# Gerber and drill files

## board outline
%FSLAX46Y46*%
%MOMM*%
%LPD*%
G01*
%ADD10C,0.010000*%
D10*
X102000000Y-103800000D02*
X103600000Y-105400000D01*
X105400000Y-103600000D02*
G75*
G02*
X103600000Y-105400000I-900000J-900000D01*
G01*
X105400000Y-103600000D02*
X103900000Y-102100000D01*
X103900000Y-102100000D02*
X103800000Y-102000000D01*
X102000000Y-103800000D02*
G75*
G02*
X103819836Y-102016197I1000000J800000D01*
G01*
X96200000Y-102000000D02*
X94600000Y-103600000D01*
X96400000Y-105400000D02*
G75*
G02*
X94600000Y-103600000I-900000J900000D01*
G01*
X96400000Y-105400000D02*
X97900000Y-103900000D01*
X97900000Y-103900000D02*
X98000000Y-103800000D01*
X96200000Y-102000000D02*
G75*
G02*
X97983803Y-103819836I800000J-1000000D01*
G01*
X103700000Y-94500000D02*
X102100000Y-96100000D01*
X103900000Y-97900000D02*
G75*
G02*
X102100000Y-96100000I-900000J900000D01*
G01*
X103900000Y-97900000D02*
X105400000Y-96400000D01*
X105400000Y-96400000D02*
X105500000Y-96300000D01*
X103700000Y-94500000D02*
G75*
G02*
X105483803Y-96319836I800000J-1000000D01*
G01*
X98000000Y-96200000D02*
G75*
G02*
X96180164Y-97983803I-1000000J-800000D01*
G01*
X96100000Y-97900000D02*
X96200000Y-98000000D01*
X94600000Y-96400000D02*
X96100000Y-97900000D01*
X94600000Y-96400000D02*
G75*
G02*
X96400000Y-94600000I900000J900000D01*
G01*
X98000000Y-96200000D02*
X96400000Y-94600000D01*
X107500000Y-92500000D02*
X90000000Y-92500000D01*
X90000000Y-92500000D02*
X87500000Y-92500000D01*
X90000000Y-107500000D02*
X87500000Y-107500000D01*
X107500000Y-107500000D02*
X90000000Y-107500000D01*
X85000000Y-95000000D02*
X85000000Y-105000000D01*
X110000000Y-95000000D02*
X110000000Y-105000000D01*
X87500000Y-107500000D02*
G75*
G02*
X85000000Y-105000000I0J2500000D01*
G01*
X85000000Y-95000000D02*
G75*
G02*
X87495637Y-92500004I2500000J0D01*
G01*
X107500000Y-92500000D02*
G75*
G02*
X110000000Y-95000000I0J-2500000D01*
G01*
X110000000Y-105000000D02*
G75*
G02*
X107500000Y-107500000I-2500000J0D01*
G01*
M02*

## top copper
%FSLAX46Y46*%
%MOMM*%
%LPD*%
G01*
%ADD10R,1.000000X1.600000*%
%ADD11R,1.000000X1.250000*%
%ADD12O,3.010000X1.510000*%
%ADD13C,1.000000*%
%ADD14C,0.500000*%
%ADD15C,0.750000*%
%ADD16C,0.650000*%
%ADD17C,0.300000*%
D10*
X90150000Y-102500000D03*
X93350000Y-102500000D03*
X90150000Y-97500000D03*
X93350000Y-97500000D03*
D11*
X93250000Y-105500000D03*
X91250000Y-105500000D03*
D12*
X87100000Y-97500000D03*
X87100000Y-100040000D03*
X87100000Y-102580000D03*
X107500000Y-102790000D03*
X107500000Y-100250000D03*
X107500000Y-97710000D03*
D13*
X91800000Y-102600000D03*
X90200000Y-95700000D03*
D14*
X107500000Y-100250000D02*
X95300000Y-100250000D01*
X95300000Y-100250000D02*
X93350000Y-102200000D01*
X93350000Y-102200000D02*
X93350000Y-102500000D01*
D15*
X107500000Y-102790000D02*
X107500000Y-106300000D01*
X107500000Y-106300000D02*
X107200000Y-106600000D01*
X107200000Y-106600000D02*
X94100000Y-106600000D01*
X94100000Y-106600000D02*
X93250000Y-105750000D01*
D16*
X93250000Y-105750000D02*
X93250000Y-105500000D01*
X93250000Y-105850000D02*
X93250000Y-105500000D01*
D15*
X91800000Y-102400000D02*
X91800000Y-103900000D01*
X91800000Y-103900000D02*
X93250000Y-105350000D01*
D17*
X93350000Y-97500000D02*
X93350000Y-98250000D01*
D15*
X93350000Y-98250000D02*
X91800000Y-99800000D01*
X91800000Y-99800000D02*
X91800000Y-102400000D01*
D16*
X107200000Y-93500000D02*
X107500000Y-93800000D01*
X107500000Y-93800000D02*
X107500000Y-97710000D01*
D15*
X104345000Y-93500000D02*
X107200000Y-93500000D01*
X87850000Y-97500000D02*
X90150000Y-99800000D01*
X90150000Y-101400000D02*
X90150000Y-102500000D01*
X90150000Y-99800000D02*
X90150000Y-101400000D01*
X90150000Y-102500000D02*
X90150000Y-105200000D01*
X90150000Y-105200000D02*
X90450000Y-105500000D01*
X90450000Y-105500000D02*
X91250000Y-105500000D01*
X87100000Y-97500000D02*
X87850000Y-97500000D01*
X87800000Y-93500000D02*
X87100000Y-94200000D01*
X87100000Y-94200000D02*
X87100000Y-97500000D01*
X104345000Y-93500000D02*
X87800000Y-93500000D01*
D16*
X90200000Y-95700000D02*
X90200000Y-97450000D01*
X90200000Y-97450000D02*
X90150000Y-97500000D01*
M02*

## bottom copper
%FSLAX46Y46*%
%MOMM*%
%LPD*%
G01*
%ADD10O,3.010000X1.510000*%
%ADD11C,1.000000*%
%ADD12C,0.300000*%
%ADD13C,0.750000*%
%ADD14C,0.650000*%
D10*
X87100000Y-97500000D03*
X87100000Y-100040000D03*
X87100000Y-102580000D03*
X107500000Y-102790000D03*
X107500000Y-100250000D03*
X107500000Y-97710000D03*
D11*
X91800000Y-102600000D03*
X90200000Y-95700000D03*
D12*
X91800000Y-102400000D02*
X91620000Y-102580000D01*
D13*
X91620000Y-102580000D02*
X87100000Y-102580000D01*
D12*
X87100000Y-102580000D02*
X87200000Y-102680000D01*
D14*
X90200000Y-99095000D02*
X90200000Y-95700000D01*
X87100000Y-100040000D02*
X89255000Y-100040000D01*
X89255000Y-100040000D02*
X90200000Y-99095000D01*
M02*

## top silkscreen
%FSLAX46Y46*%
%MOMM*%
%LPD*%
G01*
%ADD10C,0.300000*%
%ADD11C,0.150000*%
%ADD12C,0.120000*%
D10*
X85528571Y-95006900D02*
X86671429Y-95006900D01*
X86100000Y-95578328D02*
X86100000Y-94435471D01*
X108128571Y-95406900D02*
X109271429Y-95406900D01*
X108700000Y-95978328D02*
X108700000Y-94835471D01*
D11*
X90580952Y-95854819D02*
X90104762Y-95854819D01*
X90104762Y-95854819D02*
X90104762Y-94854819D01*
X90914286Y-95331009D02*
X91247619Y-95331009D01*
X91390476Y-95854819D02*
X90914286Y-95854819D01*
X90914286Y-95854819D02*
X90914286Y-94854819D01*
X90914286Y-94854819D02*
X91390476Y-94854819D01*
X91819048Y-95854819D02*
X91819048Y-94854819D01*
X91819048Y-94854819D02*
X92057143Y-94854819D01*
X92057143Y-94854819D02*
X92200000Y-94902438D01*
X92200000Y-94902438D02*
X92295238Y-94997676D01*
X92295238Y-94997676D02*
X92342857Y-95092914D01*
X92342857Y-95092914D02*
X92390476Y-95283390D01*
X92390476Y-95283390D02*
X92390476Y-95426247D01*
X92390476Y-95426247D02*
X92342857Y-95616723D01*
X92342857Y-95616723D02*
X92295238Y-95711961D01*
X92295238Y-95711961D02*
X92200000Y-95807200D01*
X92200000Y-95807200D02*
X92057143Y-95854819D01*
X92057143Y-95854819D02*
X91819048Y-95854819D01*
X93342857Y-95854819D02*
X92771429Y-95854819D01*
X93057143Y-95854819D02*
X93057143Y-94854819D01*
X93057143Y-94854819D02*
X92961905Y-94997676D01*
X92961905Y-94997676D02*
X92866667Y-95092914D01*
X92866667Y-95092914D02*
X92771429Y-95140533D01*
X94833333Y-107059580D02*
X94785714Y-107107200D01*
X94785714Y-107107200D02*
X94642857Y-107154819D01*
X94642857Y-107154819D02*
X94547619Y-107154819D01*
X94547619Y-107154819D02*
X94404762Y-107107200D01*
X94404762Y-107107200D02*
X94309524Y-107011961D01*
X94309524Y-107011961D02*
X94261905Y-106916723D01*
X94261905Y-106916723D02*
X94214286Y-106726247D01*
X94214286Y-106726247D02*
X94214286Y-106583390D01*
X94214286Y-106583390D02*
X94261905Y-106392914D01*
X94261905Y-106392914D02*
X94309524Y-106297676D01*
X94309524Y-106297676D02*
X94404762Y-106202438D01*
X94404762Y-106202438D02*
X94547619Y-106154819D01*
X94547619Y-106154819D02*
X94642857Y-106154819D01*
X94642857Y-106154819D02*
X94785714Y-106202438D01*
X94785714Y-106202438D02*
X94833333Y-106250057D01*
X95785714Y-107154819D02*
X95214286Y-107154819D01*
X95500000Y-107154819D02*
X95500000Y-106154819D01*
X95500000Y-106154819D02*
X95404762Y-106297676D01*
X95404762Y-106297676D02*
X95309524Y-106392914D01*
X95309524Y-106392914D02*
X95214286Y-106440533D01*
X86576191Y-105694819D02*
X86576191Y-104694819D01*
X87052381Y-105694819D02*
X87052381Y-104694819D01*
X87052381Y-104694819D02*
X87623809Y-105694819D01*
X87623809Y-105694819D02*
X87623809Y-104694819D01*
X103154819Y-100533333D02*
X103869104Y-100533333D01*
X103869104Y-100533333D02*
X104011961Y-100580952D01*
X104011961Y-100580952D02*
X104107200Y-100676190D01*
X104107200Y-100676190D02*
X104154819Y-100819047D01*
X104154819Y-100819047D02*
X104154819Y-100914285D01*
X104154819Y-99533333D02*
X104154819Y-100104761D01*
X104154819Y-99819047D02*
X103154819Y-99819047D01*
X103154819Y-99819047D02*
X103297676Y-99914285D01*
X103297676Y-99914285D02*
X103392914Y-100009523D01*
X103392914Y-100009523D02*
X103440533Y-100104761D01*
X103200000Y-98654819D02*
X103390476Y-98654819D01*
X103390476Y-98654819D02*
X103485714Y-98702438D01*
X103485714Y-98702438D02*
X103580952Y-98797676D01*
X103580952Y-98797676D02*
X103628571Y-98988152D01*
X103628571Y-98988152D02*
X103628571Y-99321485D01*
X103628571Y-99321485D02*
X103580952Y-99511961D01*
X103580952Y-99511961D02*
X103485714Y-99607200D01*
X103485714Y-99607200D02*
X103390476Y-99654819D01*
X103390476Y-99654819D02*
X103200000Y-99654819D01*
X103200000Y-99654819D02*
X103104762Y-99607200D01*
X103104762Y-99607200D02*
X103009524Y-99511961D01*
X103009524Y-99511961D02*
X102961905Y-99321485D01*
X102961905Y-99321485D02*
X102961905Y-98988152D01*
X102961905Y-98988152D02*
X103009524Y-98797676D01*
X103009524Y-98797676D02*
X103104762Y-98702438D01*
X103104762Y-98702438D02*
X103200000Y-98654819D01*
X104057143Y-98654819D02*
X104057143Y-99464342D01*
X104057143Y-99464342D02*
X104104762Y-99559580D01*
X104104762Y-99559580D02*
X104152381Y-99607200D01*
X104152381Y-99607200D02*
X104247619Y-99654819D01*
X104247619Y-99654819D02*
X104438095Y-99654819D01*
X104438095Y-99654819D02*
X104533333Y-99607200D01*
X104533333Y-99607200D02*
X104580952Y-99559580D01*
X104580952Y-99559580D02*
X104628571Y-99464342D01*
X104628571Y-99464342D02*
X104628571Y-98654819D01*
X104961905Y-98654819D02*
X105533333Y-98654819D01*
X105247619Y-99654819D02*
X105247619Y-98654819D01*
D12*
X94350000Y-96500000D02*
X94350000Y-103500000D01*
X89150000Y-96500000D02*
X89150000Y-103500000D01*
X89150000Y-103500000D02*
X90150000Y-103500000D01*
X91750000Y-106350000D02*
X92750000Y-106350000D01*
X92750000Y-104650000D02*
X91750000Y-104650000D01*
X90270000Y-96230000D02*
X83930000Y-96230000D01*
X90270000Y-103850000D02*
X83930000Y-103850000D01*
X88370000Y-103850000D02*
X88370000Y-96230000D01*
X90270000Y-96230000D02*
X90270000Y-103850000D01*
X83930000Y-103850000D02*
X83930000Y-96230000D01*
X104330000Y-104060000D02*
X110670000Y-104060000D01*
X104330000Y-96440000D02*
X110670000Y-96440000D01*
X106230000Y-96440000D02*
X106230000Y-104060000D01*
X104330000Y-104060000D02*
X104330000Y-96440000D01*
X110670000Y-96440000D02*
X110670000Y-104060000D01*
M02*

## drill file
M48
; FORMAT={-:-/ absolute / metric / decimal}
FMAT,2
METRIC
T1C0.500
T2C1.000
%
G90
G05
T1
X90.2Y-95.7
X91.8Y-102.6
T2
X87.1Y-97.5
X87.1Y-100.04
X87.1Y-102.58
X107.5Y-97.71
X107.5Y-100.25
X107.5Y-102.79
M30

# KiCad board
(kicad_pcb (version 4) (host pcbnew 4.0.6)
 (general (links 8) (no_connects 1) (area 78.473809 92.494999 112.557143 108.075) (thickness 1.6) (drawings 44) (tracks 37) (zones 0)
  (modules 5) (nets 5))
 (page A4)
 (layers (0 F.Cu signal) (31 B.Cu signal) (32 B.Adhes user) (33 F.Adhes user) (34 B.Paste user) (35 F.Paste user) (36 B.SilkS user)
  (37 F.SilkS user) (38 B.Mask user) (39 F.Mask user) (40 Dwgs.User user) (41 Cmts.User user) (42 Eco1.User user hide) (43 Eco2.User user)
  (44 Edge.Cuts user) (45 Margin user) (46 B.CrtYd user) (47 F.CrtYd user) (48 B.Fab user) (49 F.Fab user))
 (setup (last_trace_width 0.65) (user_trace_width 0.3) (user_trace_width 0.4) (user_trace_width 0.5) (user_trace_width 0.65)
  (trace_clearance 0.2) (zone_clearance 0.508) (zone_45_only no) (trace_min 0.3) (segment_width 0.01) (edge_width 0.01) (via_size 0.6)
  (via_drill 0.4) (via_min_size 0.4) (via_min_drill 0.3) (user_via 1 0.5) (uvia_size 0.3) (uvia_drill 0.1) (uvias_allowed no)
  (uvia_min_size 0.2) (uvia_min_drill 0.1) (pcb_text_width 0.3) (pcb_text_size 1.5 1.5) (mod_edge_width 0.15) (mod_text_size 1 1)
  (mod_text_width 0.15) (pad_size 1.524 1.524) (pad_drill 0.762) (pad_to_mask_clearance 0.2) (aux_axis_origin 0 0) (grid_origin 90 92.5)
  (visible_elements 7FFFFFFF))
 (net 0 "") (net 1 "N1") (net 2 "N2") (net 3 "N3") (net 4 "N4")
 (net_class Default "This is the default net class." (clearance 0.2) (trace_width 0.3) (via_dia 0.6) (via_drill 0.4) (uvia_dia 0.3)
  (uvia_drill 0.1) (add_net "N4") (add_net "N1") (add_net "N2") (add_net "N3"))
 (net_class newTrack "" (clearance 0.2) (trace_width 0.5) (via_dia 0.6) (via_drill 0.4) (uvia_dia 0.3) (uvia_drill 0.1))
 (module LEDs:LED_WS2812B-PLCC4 (layer F.Cu) (at 91.75 100 270)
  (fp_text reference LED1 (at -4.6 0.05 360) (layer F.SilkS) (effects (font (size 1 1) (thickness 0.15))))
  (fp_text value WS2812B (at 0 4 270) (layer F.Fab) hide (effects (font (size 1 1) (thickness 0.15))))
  (fp_line (start -3.5 -2.6) (end 3.5 -2.6) (layer F.SilkS) (width 0.12))
  (fp_line (start -3.5 2.6) (end 3.5 2.6) (layer F.SilkS) (width 0.12))
  (fp_line (start 3.5 2.6) (end 3.5 1.6) (layer F.SilkS) (width 0.12))
  (pad 3 smd rect (at 2.5 1.6 270) (size 1.6 1) (layers F.Cu F.Paste F.Mask) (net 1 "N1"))
  (pad 4 smd rect (at 2.5 -1.6 270) (size 1.6 1) (layers F.Cu F.Paste F.Mask) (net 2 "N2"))
  (pad 2 smd rect (at -2.5 1.6 270) (size 1.6 1) (layers F.Cu F.Paste F.Mask) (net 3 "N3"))
  (pad 1 smd rect (at -2.5 -1.6 270) (size 1.6 1) (layers F.Cu F.Paste F.Mask) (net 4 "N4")))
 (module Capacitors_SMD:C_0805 (layer F.Cu) (at 92.25 105.5 180)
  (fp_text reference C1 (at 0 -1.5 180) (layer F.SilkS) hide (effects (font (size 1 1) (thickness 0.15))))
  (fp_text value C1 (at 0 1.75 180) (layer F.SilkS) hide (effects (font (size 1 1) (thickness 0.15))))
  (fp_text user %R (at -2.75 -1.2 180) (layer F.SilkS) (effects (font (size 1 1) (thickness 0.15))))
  (fp_line (start 0.5 -0.85) (end -0.5 -0.85) (layer F.SilkS) (width 0.12))
  (fp_line (start -0.5 0.85) (end 0.5 0.85) (layer F.SilkS) (width 0.12))
  (pad 1 smd rect (at -1 0 180) (size 1 1.25) (layers F.Cu F.Paste F.Mask) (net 4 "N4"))
  (pad 2 smd rect (at 1 0 180) (size 1 1.25) (layers F.Cu F.Paste F.Mask) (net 1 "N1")))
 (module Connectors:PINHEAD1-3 (layer F.Cu) (at 87.1 97.5 270)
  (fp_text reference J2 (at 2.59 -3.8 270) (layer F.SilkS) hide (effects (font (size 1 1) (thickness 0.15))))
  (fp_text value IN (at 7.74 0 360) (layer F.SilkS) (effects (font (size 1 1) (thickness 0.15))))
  (fp_line (start -1.27 -3.17) (end -1.27 3.17) (layer F.SilkS) (width 0.12))
  (fp_line (start 6.35 -3.17) (end 6.35 3.17) (layer F.SilkS) (width 0.12))
  (fp_line (start 6.35 -1.27) (end -1.27 -1.27) (layer F.SilkS) (width 0.12))
  (fp_line (start -1.27 -3.17) (end 6.35 -3.17) (layer F.SilkS) (width 0.12))
  (fp_line (start 6.35 3.17) (end -1.27 3.17) (layer F.SilkS) (width 0.12))
  (pad 1 thru_hole oval (at 0 0 270) (size 1.51 3.01) (drill 1) (layers *.Cu *.Mask) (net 1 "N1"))
  (pad 2 thru_hole oval (at 2.54 0 270) (size 1.51 3.01) (drill 1) (layers *.Cu *.Mask) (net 3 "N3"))
  (pad 3 thru_hole oval (at 5.08 0 270) (size 1.51 3.01) (drill 1) (layers *.Cu *.Mask) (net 4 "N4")))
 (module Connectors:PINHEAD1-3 (layer F.Cu) (at 107.5 102.79 90)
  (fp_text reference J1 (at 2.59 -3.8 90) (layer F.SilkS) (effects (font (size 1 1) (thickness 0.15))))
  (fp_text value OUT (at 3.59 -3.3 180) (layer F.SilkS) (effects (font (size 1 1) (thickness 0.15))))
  (fp_line (start -1.27 -3.17) (end -1.27 3.17) (layer F.SilkS) (width 0.12))
  (fp_line (start 6.35 -3.17) (end 6.35 3.17) (layer F.SilkS) (width 0.12))
  (fp_line (start 6.35 -1.27) (end -1.27 -1.27) (layer F.SilkS) (width 0.12))
  (fp_line (start -1.27 -3.17) (end 6.35 -3.17) (layer F.SilkS) (width 0.12))
  (fp_line (start 6.35 3.17) (end -1.27 3.17) (layer F.SilkS) (width 0.12))
  (pad 1 thru_hole oval (at 0 0 90) (size 1.51 3.01) (drill 1) (layers *.Cu *.Mask) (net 4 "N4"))
  (pad 2 thru_hole oval (at 2.54 0 90) (size 1.51 3.01) (drill 1) (layers *.Cu *.Mask) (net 2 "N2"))
  (pad 3 thru_hole oval (at 5.08 0 90) (size 1.51 3.01) (drill 1) (layers *.Cu *.Mask) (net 1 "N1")))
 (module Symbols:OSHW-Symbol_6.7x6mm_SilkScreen (layer B.Cu) (at 92.9 100.1 180)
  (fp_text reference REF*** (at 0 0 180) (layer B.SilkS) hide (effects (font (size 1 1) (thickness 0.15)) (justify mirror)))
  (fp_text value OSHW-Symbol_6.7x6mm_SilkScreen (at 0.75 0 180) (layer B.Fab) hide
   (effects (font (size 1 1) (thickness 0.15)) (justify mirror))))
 (gr_line (start 102 103.8) (end 103.6 105.4) (layer Edge.Cuts) (width 0.01))
 (gr_arc (start 104.5 104.5) (end 105.4 103.6) (angle 180) (layer Edge.Cuts) (width 0.01))
 (gr_line (start 105.4 103.6) (end 103.9 102.1) (layer Edge.Cuts) (width 0.01))
 (gr_line (start 103.9 102.1) (end 103.8 102) (layer Edge.Cuts) (width 0.01))
 (gr_arc (start 103 103) (end 102 103.8) (angle 168.4653793) (layer Edge.Cuts) (width 0.01))
 (gr_line (start 96.2 102) (end 94.6 103.6) (layer Edge.Cuts) (width 0.01))
 (gr_arc (start 95.5 104.5) (end 96.4 105.4) (angle 180) (layer Edge.Cuts) (width 0.01))
 (gr_line (start 96.4 105.4) (end 97.9 103.9) (layer Edge.Cuts) (width 0.01))
 (gr_line (start 97.9 103.9) (end 98 103.8) (layer Edge.Cuts) (width 0.01))
 (gr_arc (start 97 103) (end 96.2 102) (angle 168.4653793) (layer Edge.Cuts) (width 0.01))
 (gr_line (start 103.7 94.5) (end 102.1 96.1) (layer Edge.Cuts) (width 0.01))
 (gr_arc (start 103 97) (end 103.9 97.9) (angle 180) (layer Edge.Cuts) (width 0.01))
 (gr_line (start 103.9 97.9) (end 105.4 96.4) (layer Edge.Cuts) (width 0.01))
 (gr_line (start 105.4 96.4) (end 105.5 96.3) (layer Edge.Cuts) (width 0.01))
 (gr_arc (start 104.5 95.5) (end 103.7 94.5) (angle 168.4653793) (layer Edge.Cuts) (width 0.01))
 (gr_arc (start 97 97) (end 98 96.2) (angle 168.4653793) (layer Edge.Cuts) (width 0.01))
 (gr_line (start 96.1 97.9) (end 96.2 98) (layer Edge.Cuts) (width 0.01))
 (gr_line (start 94.6 96.4) (end 96.1 97.9) (layer Edge.Cuts) (width 0.01))
 (gr_arc (start 95.5 95.5) (end 94.6 96.4) (angle 180) (layer Edge.Cuts) (width 0.01))
 (gr_line (start 98 96.2) (end 96.4 94.6) (layer Edge.Cuts) (width 0.01))
 (gr_line (start 107.5 92.5) (end 90 92.5) (layer Edge.Cuts) (width 0.01))
 (gr_line (start 90 92.5) (end 87.5 92.5) (layer Edge.Cuts) (width 0.01))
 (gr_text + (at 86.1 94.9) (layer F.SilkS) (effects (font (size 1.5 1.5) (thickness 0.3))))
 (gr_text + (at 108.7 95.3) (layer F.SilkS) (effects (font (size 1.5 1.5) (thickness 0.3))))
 (gr_line (start 90 107.5) (end 87.5 107.5) (layer Edge.Cuts) (width 0.01))
 (gr_line (start 107.5 107.5) (end 90 107.5) (layer Edge.Cuts) (width 0.01))
 (gr_line (start 85 95) (end 85 105) (layer Edge.Cuts) (width 0.01))
 (gr_line (start 110 95) (end 110 105) (layer Edge.Cuts) (width 0.01))
 (gr_arc (start 87.5 105) (end 87.5 107.5) (angle 90) (layer Edge.Cuts) (width 0.01))
 (gr_arc (start 87.5 95) (end 85 95) (angle 89.9) (layer Edge.Cuts) (width 0.01))
 (gr_arc (start 107.5 95) (end 107.5 92.5) (angle 90) (layer Edge.Cuts) (width 0.01))
 (gr_arc (start 107.5 105) (end 110 105) (angle 90) (layer Edge.Cuts) (width 0.01))
 (segment (start 107.5 100.25) (end 95.3 100.25) (width 0.5) (layer F.Cu) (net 2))
 (segment (start 95.3 100.25) (end 93.35 102.2) (width 0.5) (layer F.Cu) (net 2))
 (segment (start 93.35 102.2) (end 93.35 102.5) (width 0.5) (layer F.Cu) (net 2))
 (segment (start 107.5 102.79) (end 107.5 106.3) (width 0.75) (layer F.Cu) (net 4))
 (segment (start 107.5 106.3) (end 107.2 106.6) (width 0.75) (layer F.Cu) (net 4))
 (segment (start 107.2 106.6) (end 94.1 106.6) (width 0.75) (layer F.Cu) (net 4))
 (segment (start 94.1 106.6) (end 93.25 105.75) (width 0.75) (layer F.Cu) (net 4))
 (segment (start 93.25 105.75) (end 93.25 105.5) (width 0.65) (layer F.Cu) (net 4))
 (segment (start 93.25 105.85) (end 93.25 105.5) (width 0.65) (layer F.Cu) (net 4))
 (segment (start 91.8 102.4) (end 91.8 103.9) (width 0.75) (layer F.Cu) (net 4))
 (segment (start 91.8 103.9) (end 93.25 105.35) (width 0.75) (layer F.Cu) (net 4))
 (segment (start 93.35 97.5) (end 93.35 98.25) (width 0.3) (layer F.Cu) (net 4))
 (segment (start 93.35 98.25) (end 91.8 99.8) (width 0.75) (layer F.Cu) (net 4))
 (segment (start 91.8 99.8) (end 91.8 102.4) (width 0.75) (layer F.Cu) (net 4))
 (via (at 91.8 102.6) (size 1) (drill 0.5) (layers F.Cu B.Cu) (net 4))
 (segment (start 91.8 102.4) (end 91.62 102.58) (width 0.3) (layer B.Cu) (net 4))
 (segment (start 91.62 102.58) (end 87.1 102.58) (width 0.75) (layer B.Cu) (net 4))
 (segment (start 87.1 102.58) (end 87.2 102.68) (width 0.3) (layer B.Cu) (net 4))
 (segment (start 107.2 93.5) (end 107.5 93.8) (width 0.65) (layer F.Cu) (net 1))
 (segment (start 107.5 93.8) (end 107.5 97.71) (width 0.65) (layer F.Cu) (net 1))
 (segment (start 104.345 93.5) (end 107.2 93.5) (width 0.75) (layer F.Cu) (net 1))
 (segment (start 87.85 97.5) (end 90.15 99.8) (width 0.75) (layer F.Cu) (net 1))
 (segment (start 90.15 101.4) (end 90.15 102.5) (width 0.75) (layer F.Cu) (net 1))
 (segment (start 90.15 99.8) (end 90.15 101.4) (width 0.75) (layer F.Cu) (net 1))
 (segment (start 90.15 102.5) (end 90.15 105.2) (width 0.75) (layer F.Cu) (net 1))
 (segment (start 90.15 105.2) (end 90.45 105.5) (width 0.75) (layer F.Cu) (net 1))
 (segment (start 90.45 105.5) (end 91.25 105.5) (width 0.75) (layer F.Cu) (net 1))
 (segment (start 87.1 97.5) (end 87.85 97.5) (width 0.75) (layer F.Cu) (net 1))
 (segment (start 87.8 93.5) (end 87.1 94.2) (width 0.75) (layer F.Cu) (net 1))
 (segment (start 87.1 94.2) (end 87.1 97.5) (width 0.75) (layer F.Cu) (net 1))
 (segment (start 104.345 93.5) (end 87.8 93.5) (width 0.75) (layer F.Cu) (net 1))
 (segment (start 90.2 95.7) (end 90.2 97.45) (width 0.65) (layer F.Cu) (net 3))
 (segment (start 90.2 97.45) (end 90.15 97.5) (width 0.65) (layer F.Cu) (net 3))
 (segment (start 90.2 99.095) (end 90.2 95.7) (width 0.65) (layer B.Cu) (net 3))
 (via (at 90.2 95.7) (size 1) (drill 0.5) (layers F.Cu B.Cu) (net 3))
 (segment (start 87.1 100.04) (end 89.255 100.04) (width 0.65) (layer B.Cu) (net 3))
 (segment (start 89.255 100.04) (end 90.2 99.095) (width 0.65) (layer B.Cu) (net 3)))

